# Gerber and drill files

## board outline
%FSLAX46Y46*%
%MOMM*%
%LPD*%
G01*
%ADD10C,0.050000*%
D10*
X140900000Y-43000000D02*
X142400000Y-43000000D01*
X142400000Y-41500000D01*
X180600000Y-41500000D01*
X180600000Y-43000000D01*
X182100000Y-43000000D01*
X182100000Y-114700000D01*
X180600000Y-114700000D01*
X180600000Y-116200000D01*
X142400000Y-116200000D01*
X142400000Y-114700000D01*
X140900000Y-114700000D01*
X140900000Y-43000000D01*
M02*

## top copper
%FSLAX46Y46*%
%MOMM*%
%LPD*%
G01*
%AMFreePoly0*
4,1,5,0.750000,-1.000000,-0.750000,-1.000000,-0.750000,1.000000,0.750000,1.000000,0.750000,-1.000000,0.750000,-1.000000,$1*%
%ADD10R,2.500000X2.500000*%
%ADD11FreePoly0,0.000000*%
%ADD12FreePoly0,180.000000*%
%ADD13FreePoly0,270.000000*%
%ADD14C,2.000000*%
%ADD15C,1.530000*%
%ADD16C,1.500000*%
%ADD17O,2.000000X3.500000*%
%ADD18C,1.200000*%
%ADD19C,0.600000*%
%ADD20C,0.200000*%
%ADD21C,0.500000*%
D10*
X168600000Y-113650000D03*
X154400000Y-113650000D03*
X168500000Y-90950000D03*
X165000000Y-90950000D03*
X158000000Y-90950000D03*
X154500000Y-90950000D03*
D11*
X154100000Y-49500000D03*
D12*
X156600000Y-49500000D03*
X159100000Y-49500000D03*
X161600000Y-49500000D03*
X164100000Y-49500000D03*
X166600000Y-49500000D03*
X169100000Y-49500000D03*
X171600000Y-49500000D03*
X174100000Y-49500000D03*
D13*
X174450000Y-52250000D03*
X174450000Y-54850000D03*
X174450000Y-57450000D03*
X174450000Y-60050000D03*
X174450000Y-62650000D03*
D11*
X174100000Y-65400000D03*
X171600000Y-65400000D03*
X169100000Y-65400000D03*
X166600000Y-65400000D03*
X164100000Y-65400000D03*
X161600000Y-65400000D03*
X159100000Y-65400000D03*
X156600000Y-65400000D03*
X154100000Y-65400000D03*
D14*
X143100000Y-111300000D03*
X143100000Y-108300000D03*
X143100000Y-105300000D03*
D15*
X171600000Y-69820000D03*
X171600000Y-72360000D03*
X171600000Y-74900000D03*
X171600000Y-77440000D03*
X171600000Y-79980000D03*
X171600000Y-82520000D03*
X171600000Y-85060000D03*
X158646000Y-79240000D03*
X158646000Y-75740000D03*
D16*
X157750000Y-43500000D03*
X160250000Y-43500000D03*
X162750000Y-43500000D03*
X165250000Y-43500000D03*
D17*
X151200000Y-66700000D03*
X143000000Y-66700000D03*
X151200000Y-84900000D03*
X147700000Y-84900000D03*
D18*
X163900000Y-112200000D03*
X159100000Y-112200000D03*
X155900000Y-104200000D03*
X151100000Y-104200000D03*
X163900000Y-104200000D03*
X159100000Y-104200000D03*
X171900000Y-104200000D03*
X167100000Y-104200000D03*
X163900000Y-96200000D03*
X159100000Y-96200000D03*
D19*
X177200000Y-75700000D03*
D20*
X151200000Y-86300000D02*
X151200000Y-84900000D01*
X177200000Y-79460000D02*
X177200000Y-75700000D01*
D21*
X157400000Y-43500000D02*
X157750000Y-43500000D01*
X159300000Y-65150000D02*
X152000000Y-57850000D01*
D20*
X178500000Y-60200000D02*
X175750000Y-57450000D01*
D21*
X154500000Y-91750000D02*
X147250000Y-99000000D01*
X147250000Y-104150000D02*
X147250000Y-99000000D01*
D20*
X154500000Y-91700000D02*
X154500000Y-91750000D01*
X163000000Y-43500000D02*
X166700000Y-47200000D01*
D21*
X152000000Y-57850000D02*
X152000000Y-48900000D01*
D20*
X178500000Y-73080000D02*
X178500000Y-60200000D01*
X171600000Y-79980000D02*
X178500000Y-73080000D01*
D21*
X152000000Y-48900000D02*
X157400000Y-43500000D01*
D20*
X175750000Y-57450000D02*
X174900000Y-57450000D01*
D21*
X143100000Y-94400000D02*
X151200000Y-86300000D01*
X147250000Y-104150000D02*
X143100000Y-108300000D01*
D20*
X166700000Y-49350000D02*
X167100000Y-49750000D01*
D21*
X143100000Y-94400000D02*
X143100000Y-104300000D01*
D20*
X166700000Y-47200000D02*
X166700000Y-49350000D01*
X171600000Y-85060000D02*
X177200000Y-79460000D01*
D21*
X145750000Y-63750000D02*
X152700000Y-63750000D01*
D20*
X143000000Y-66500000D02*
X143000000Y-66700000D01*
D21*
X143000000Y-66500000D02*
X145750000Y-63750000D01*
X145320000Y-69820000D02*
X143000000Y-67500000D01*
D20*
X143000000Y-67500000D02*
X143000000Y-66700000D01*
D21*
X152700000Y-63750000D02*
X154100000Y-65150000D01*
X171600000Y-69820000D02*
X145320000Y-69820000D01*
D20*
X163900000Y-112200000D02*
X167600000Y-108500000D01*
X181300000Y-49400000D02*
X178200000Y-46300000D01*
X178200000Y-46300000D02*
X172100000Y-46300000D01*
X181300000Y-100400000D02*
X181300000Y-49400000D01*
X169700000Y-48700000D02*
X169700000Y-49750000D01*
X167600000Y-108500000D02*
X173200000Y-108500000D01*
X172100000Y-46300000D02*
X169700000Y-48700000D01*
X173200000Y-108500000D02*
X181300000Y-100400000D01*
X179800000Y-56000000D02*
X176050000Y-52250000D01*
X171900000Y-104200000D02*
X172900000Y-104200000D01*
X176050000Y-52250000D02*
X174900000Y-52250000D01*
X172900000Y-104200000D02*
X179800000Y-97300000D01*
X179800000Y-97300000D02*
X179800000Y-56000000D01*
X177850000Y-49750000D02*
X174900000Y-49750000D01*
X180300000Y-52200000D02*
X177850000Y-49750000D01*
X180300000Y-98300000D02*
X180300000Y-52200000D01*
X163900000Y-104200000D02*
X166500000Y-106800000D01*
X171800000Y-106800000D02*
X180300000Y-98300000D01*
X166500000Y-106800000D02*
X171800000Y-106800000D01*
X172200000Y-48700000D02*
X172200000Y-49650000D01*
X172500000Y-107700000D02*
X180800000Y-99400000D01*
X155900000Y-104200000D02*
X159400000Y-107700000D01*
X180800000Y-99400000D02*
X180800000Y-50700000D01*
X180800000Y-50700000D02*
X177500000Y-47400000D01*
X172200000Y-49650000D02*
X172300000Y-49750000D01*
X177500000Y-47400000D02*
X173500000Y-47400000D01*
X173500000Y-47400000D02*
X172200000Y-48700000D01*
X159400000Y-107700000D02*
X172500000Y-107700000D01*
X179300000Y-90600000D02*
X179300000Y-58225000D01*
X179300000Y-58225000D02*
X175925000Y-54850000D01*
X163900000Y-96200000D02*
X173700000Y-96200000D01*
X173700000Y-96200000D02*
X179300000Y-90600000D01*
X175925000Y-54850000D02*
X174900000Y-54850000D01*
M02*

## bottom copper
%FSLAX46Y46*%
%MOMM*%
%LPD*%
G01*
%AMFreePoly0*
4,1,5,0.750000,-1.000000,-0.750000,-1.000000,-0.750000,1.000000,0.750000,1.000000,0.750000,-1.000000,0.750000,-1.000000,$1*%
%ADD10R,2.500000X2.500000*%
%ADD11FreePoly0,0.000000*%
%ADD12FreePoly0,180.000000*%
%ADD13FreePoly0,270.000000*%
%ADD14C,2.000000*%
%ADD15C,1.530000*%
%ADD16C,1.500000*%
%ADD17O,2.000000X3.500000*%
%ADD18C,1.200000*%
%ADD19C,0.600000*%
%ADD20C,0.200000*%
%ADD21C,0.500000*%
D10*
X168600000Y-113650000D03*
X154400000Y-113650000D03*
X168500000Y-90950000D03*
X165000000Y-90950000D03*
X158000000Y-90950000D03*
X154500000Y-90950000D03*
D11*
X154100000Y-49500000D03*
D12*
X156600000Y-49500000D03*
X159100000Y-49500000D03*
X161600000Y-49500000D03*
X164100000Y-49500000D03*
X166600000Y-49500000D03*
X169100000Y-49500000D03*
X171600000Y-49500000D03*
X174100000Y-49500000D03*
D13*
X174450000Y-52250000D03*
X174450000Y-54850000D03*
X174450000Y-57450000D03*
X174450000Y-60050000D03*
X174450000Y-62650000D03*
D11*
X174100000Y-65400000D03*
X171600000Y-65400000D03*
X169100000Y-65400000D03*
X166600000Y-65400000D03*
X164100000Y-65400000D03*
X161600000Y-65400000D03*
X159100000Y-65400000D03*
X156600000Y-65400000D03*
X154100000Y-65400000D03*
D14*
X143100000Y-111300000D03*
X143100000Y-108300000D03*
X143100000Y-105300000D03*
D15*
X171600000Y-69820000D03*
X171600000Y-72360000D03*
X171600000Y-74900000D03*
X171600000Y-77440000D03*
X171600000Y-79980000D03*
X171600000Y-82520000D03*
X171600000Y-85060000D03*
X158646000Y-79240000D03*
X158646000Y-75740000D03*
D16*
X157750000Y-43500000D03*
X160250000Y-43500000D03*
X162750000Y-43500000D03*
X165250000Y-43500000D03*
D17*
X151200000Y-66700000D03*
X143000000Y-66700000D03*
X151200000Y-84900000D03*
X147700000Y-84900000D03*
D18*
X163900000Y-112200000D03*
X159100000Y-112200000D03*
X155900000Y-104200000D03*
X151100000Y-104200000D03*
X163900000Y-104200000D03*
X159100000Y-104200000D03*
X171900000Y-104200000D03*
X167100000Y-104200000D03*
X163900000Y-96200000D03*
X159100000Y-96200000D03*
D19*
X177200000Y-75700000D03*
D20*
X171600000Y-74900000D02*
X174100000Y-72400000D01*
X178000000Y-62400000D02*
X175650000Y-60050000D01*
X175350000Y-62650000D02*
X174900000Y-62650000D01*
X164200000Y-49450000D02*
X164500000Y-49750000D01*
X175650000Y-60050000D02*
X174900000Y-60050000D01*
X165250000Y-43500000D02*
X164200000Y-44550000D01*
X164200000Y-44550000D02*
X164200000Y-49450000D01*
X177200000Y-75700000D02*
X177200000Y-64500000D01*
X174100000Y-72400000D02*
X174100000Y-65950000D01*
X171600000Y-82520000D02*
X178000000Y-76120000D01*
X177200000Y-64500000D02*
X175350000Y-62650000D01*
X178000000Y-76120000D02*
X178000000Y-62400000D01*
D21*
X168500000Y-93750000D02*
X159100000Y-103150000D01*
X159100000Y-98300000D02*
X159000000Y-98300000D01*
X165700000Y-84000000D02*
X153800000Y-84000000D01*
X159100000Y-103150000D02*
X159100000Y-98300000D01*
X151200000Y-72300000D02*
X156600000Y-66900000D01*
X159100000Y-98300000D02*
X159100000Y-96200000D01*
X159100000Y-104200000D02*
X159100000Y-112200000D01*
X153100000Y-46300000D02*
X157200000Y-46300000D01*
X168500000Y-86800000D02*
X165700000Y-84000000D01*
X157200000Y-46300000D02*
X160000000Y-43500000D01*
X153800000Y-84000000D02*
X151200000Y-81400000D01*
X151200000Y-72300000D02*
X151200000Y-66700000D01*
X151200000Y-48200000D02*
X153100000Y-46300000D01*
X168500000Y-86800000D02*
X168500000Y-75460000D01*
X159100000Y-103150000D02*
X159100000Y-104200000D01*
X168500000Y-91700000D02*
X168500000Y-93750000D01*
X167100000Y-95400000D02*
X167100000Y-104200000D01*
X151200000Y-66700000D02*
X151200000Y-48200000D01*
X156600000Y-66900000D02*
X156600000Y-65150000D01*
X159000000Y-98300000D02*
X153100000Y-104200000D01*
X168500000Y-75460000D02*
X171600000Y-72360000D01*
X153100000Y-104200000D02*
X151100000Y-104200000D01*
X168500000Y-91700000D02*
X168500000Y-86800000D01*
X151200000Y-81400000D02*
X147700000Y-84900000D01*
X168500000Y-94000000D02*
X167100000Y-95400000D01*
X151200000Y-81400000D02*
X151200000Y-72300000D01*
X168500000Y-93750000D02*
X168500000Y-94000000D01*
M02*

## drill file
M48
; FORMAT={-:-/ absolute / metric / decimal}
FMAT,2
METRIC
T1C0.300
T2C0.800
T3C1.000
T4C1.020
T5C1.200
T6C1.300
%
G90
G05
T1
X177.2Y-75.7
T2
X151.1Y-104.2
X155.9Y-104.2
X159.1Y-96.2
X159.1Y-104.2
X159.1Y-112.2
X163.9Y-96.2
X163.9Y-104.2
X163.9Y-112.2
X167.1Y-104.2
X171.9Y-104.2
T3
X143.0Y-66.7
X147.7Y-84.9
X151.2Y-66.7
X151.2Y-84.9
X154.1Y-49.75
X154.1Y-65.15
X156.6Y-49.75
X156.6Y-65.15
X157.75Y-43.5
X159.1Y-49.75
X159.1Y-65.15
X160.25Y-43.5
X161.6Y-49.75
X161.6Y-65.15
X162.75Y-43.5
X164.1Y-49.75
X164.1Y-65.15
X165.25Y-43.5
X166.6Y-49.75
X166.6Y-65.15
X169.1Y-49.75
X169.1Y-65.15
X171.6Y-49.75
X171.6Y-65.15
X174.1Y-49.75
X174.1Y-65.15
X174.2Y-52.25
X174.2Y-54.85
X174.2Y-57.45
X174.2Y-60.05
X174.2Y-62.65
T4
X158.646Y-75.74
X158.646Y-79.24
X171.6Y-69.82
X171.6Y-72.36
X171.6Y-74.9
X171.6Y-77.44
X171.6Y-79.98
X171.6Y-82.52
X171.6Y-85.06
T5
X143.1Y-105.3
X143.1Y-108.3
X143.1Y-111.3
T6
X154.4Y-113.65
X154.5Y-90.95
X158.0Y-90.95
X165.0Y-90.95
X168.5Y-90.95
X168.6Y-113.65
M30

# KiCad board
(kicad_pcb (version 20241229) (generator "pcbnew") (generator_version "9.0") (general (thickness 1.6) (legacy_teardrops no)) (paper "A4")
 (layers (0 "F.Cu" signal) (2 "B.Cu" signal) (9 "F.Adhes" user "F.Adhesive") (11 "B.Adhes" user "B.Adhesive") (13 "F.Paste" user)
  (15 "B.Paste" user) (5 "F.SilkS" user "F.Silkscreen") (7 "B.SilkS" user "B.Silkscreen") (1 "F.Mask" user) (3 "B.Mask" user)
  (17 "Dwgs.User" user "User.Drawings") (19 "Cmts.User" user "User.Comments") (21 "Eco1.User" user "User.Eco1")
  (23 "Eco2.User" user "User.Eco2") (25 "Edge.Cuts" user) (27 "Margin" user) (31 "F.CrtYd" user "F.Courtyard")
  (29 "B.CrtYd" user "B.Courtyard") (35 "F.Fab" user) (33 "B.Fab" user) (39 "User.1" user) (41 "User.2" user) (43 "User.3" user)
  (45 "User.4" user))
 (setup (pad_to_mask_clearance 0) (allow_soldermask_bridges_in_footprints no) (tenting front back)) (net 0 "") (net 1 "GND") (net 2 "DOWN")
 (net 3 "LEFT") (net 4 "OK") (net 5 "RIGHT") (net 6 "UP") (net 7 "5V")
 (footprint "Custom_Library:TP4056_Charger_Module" (layer "F.Cu") (at 161.5 101.9 180)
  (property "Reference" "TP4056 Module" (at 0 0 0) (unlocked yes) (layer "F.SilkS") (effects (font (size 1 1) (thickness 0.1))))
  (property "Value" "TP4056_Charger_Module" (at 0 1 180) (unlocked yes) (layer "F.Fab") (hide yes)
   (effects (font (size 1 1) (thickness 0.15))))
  (pad "1" thru_hole rect (at -7.1 -11.75 180) (size 2.5 2.5) (drill 1.3) (layers "*.Cu" "*.Mask") (remove_unused_layers no)
   (thermal_bridge_angle 45))
  (pad "2" thru_hole rect (at 7.1 -11.75 180) (size 2.5 2.5) (drill 1.3) (layers "*.Cu" "*.Mask") (remove_unused_layers no)
   (thermal_bridge_angle 45))
  (pad "3" thru_hole rect (at -7 10.95 180) (size 2.5 2.5) (drill 1.3) (layers "*.Cu" "*.Mask") (remove_unused_layers no) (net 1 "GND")
   (thermal_bridge_angle 45))
  (pad "4" thru_hole rect (at -3.5 10.95 180) (size 2.5 2.5) (drill 1.3) (layers "*.Cu" "*.Mask") (remove_unused_layers no)
   (thermal_bridge_angle 45))
  (pad "5" thru_hole rect (at 3.5 10.95 180) (size 2.5 2.5) (drill 1.3) (layers "*.Cu" "*.Mask") (remove_unused_layers no)
   (thermal_bridge_angle 45))
  (pad "6" thru_hole rect (at 7 10.95 180) (size 2.5 2.5) (drill 1.3) (layers "*.Cu" "*.Mask") (remove_unused_layers no)
   (thermal_bridge_angle 45))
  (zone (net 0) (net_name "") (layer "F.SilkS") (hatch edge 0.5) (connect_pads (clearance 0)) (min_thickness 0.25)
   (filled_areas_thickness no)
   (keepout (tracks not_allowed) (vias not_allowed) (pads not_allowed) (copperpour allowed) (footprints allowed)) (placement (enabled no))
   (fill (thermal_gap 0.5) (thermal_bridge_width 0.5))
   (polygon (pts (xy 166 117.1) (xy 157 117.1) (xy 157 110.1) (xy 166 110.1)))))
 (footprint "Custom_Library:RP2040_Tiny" (layer "F.Cu") (at 164.5 57.45)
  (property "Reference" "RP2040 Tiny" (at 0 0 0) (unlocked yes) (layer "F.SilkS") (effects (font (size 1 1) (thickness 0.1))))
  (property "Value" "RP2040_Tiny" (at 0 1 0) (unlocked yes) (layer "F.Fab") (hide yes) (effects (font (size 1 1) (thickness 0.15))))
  (pad "1" thru_hole custom (at -10.4 -7.7) (size 1.5 2) (drill 1 (offset 0 -0.25)) (layers "*.Cu" "*.Mask") (remove_unused_layers no)
   (options (clearance outline) (anchor rect)) (primitives))
  (pad "2" thru_hole custom (at -7.9 -7.7 180) (size 1.5 2) (drill 1 (offset 0 0.25)) (layers "*.Cu" "*.Mask") (remove_unused_layers no)
   (options (clearance outline) (anchor rect)) (primitives))
  (pad "3" thru_hole custom (at -5.4 -7.7 180) (size 1.5 2) (drill 1 (offset 0 0.25)) (layers "*.Cu" "*.Mask") (remove_unused_layers no)
   (options (clearance outline) (anchor rect)) (primitives))
  (pad "4" thru_hole custom (at -2.9 -7.7 180) (size 1.5 2) (drill 1 (offset 0 0.25)) (layers "*.Cu" "*.Mask") (remove_unused_layers no)
   (options (clearance outline) (anchor rect)) (primitives))
  (pad "5" thru_hole custom (at -0.4 -7.7 180) (size 1.5 2) (drill 1 (offset 0 0.25)) (layers "*.Cu" "*.Mask") (remove_unused_layers no)
   (options (clearance outline) (anchor rect)) (primitives))
  (pad "6" thru_hole custom (at 2.1 -7.7 180) (size 1.5 2) (drill 1 (offset 0 0.25)) (layers "*.Cu" "*.Mask") (remove_unused_layers no)
   (options (clearance outline) (anchor rect)) (primitives))
  (pad "7" thru_hole custom (at 4.6 -7.7 180) (size 1.5 2) (drill 1 (offset 0 0.25)) (layers "*.Cu" "*.Mask") (remove_unused_layers no)
   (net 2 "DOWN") (options (clearance outline) (anchor rect)) (primitives))
  (pad "8" thru_hole custom (at 7.1 -7.7 180) (size 1.5 2) (drill 1 (offset 0 0.25)) (layers "*.Cu" "*.Mask") (remove_unused_layers no)
   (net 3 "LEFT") (options (clearance outline) (anchor rect)) (primitives))
  (pad "9" thru_hole custom (at 9.6 -7.7 180) (size 1.5 2) (drill 1 (offset 0 0.25)) (layers "*.Cu" "*.Mask") (remove_unused_layers no)
   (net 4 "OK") (options (clearance outline) (anchor rect)) (primitives))
  (pad "10" thru_hole custom (at 9.7 -5.2 270) (size 1.5 2) (drill 1 (offset 0 -0.25)) (layers "*.Cu" "*.Mask") (remove_unused_layers no)
   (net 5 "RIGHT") (options (clearance outline) (anchor rect)) (primitives))
  (pad "11" thru_hole custom (at 9.7 -2.6 270) (size 1.5 2) (drill 1 (offset 0 -0.25)) (layers "*.Cu" "*.Mask") (remove_unused_layers no)
   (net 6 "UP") (options (clearance outline) (anchor rect)) (primitives))
  (pad "12" thru_hole custom (at 9.7 0 270) (size 1.5 2) (drill 1 (offset 0 -0.25)) (layers "*.Cu" "*.Mask") (remove_unused_layers no)
   (options (clearance outline) (anchor rect)) (primitives))
  (pad "13" thru_hole custom (at 9.7 2.6 270) (size 1.5 2) (drill 1 (offset 0 -0.25)) (layers "*.Cu" "*.Mask") (remove_unused_layers no)
   (options (clearance outline) (anchor rect)) (primitives))
  (pad "14" thru_hole custom (at 9.7 5.2 270) (size 1.5 2) (drill 1 (offset 0 -0.25)) (layers "*.Cu" "*.Mask") (remove_unused_layers no)
   (options (clearance outline) (anchor rect)) (primitives))
  (pad "15" thru_hole custom (at 9.6 7.7) (size 1.5 2) (drill 1 (offset 0 0.25)) (layers "*.Cu" "*.Mask") (remove_unused_layers no)
   (options (clearance outline) (anchor rect)) (primitives))
  (pad "16" thru_hole custom (at 7.1 7.7) (size 1.5 2) (drill 1 (offset 0 0.25)) (layers "*.Cu" "*.Mask") (remove_unused_layers no)
   (options (clearance outline) (anchor rect)) (primitives))
  (pad "17" thru_hole custom (at 4.6 7.7) (size 1.5 2) (drill 1 (offset 0 0.25)) (layers "*.Cu" "*.Mask") (remove_unused_layers no)
   (options (clearance outline) (anchor rect)) (primitives))
  (pad "18" thru_hole custom (at 2.1 7.7) (size 1.5 2) (drill 1 (offset 0 0.25)) (layers "*.Cu" "*.Mask") (remove_unused_layers no)
   (options (clearance outline) (anchor rect)) (primitives))
  (pad "19" thru_hole custom (at -0.4 7.7) (size 1.5 2) (drill 1 (offset 0 0.25)) (layers "*.Cu" "*.Mask") (remove_unused_layers no)
   (options (clearance outline) (anchor rect)) (primitives))
  (pad "20" thru_hole custom (at -2.9 7.7) (size 1.5 2) (drill 1 (offset 0 0.25)) (layers "*.Cu" "*.Mask") (remove_unused_layers no)
   (options (clearance outline) (anchor rect)) (primitives))
  (pad "21" thru_hole custom (at -5.4 7.7) (size 1.5 2) (drill 1 (offset 0 0.25)) (layers "*.Cu" "*.Mask") (remove_unused_layers no)
   (options (clearance outline) (anchor rect)) (primitives))
  (pad "22" thru_hole custom (at -7.9 7.7) (size 1.5 2) (drill 1 (offset 0 0.25)) (layers "*.Cu" "*.Mask") (remove_unused_layers no)
   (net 1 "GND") (options (clearance outline) (anchor rect)) (primitives))
  (pad "23" thru_hole custom (at -10.4 7.7) (size 1.5 2) (drill 1 (offset 0 0.25)) (layers "*.Cu" "*.Mask") (remove_unused_layers no)
   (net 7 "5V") (options (clearance outline) (anchor rect)) (primitives))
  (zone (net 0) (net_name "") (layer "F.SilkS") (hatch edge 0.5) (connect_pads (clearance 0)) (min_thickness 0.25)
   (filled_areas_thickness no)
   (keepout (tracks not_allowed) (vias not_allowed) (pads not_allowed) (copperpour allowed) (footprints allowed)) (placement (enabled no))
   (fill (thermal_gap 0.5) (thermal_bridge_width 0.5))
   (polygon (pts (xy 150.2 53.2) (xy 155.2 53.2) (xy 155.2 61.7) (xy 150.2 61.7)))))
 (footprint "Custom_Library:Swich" (layer "F.Cu") (at 143.1 108.3 90)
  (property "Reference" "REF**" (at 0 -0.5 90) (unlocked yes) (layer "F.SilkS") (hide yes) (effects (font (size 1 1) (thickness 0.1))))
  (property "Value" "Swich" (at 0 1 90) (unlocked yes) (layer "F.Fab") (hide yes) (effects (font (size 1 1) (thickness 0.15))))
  (pad "1" thru_hole circle (at -3 0 90) (size 2 2) (drill 1.2) (layers "*.Cu" "*.Mask") (remove_unused_layers no))
  (pad "2" thru_hole circle (at 0 0 90) (size 2 2) (drill 1.2) (layers "*.Cu" "*.Mask") (remove_unused_layers no))
  (pad "3" thru_hole circle (at 3 0 90) (size 2 2) (drill 1.2) (layers "*.Cu" "*.Mask") (remove_unused_layers no)))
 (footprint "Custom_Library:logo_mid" (layer "F.Cu") (at 177.5 100 90)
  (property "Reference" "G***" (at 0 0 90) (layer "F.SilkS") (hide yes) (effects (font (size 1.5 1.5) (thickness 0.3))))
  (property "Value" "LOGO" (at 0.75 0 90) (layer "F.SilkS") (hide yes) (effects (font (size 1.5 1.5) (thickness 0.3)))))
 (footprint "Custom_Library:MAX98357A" (layer "F.Cu") (at 164.615 77.25 90)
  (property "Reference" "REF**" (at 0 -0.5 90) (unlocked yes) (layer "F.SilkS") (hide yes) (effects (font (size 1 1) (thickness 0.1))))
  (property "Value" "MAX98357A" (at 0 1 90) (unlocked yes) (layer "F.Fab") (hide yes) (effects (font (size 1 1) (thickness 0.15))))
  (pad "JP1_1" thru_hole circle (at 7.43 6.985 90) (size 1.53 1.53) (drill 1.02) (layers "*.Cu" "*.Mask") (remove_unused_layers no)
   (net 7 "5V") (solder_mask_margin 0.102))
  (pad "JP1_2" thru_hole circle (at 4.89 6.985 90) (size 1.53 1.53) (drill 1.02) (layers "*.Cu" "*.Mask") (remove_unused_layers no)
   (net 1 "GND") (solder_mask_margin 0.102))
  (pad "JP1_3" thru_hole circle (at 2.35 6.985 90) (size 1.53 1.53) (drill 1.02) (layers "*.Cu" "*.Mask") (remove_unused_layers no)
   (solder_mask_margin 0.102))
  (pad "JP1_4" thru_hole circle (at -0.19 6.985 90) (size 1.53 1.53) (drill 1.02) (layers "*.Cu" "*.Mask") (remove_unused_layers no)
   (solder_mask_margin 0.102))
  (pad "JP1_5" thru_hole circle (at -2.73 6.985 90) (size 1.53 1.53) (drill 1.02) (layers "*.Cu" "*.Mask") (remove_unused_layers no)
   (solder_mask_margin 0.102))
  (pad "JP1_6" thru_hole circle (at -5.27 6.985 90) (size 1.53 1.53) (drill 1.02) (layers "*.Cu" "*.Mask") (remove_unused_layers no)
   (solder_mask_margin 0.102))
  (pad "JP1_7" thru_hole circle (at -7.81 6.985 90) (size 1.53 1.53) (drill 1.02) (layers "*.Cu" "*.Mask") (remove_unused_layers no)
   (solder_mask_margin 0.102))
  (pad "X1_1" thru_hole circle (at -1.99 -5.969 90) (size 1.53 1.53) (drill 1.02) (layers "*.Cu" "*.Mask") (remove_unused_layers no)
   (solder_mask_margin 0.102))
  (pad "X1_2" thru_hole circle (at 1.51 -5.969 90) (size 1.53 1.53) (drill 1.02) (layers "*.Cu" "*.Mask") (remove_unused_layers no)
   (solder_mask_margin 0.102)))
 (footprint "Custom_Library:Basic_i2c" (layer "F.Cu") (at 161.5 43.5)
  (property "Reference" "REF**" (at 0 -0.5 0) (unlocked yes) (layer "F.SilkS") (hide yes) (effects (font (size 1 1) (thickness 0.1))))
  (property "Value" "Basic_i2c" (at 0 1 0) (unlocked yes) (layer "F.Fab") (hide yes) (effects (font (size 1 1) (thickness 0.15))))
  (pad "1" thru_hole circle (at -3.75 0) (size 1.5 1.5) (drill 1) (layers "*.Cu" "*.Mask") (remove_unused_layers no))
  (pad "2" thru_hole circle (at -1.25 0) (size 1.5 1.5) (drill 1) (layers "*.Cu" "*.Mask") (remove_unused_layers no) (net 1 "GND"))
  (pad "3" thru_hole circle (at 1.25 0) (size 1.5 1.5) (drill 1) (layers "*.Cu" "*.Mask") (remove_unused_layers no))
  (pad "4" thru_hole circle (at 3.75 0) (size 1.5 1.5) (drill 1) (layers "*.Cu" "*.Mask") (remove_unused_layers no)))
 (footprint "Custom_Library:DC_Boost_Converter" (layer "F.Cu") (at 147.1 75.8 -90)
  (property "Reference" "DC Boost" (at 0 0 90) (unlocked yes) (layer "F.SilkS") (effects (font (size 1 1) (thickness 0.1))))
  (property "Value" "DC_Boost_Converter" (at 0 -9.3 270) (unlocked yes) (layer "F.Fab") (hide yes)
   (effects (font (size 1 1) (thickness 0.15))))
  (pad "1" thru_hole oval (at -9.1 -4.1) (size 2 3.5) (drill 1) (layers "*.Cu" "*.Mask") (remove_unused_layers no) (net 1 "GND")
   (thermal_bridge_angle 45))
  (pad "2" thru_hole oval (at -9.1 4.1) (size 2 3.5) (drill 1) (layers "*.Cu" "*.Mask") (remove_unused_layers no) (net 7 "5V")
   (thermal_bridge_angle 45))
  (pad "3" thru_hole oval (at 9.1 -4.1) (size 2 3.5) (drill 1) (layers "*.Cu" "*.Mask") (remove_unused_layers no) (thermal_bridge_angle 45))
  (pad "4" thru_hole oval (at 9.1 -0.6) (size 2 3.5) (drill 1) (layers "*.Cu" "*.Mask") (remove_unused_layers no) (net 1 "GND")
   (thermal_bridge_angle 45)))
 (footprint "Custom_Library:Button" (layer "B.Cu") (at 161.5 112.2 180)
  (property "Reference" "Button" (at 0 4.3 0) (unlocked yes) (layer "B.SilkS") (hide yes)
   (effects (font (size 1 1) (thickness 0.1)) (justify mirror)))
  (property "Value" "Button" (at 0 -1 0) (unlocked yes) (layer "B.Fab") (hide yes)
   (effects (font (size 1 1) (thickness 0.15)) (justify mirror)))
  (pad "1" thru_hole circle (at -2.4 0 180) (size 1.2 1.2) (drill 0.8) (layers "*.Cu" "*.Mask") (remove_unused_layers no) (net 2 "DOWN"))
  (pad "2" thru_hole circle (at 2.4 0 180) (size 1.2 1.2) (drill 0.8) (layers "*.Cu" "*.Mask") (remove_unused_layers no) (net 1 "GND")))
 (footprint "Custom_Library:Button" (layer "B.Cu") (at 153.5 104.2 180)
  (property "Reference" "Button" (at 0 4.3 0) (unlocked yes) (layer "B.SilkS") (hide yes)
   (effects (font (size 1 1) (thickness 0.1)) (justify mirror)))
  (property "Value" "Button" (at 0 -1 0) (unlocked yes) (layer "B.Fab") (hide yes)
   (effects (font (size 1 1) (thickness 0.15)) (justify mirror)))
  (pad "1" thru_hole circle (at -2.4 0 180) (size 1.2 1.2) (drill 0.8) (layers "*.Cu" "*.Mask") (remove_unused_layers no) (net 3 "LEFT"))
  (pad "2" thru_hole circle (at 2.4 0 180) (size 1.2 1.2) (drill 0.8) (layers "*.Cu" "*.Mask") (remove_unused_layers no) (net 1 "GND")))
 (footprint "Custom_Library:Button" (layer "B.Cu") (at 161.5 104.2 180)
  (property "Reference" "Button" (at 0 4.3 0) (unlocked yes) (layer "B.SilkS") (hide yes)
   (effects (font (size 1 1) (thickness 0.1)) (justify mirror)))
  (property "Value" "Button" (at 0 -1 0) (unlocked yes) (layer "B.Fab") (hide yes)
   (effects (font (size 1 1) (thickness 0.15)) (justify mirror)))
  (pad "1" thru_hole circle (at -2.4 0 180) (size 1.2 1.2) (drill 0.8) (layers "*.Cu" "*.Mask") (remove_unused_layers no) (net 4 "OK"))
  (pad "2" thru_hole circle (at 2.4 0 180) (size 1.2 1.2) (drill 0.8) (layers "*.Cu" "*.Mask") (remove_unused_layers no) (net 1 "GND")))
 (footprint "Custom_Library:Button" (layer "B.Cu") (at 169.5 104.2 180)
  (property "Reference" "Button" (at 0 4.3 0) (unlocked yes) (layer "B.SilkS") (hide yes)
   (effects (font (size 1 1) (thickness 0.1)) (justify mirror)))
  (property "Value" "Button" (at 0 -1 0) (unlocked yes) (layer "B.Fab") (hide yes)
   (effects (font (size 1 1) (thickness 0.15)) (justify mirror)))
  (pad "1" thru_hole circle (at -2.4 0 180) (size 1.2 1.2) (drill 0.8) (layers "*.Cu" "*.Mask") (remove_unused_layers no) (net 5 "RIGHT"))
  (pad "2" thru_hole circle (at 2.4 0 180) (size 1.2 1.2) (drill 0.8) (layers "*.Cu" "*.Mask") (remove_unused_layers no) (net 1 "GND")))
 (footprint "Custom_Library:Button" (layer "B.Cu") (at 161.5 96.2 180)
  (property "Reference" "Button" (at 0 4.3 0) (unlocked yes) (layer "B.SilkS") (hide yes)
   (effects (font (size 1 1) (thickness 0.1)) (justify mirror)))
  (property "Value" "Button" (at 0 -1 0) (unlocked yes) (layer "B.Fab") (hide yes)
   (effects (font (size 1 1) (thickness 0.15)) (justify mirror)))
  (pad "1" thru_hole circle (at -2.4 0 180) (size 1.2 1.2) (drill 0.8) (layers "*.Cu" "*.Mask") (remove_unused_layers no) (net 6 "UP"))
  (pad "2" thru_hole circle (at 2.4 0 180) (size 1.2 1.2) (drill 0.8) (layers "*.Cu" "*.Mask") (remove_unused_layers no) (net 1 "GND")))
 (gr_poly
  (pts (xy 140.9 43) (xy 142.4 43) (xy 142.4 41.5) (xy 180.6 41.5) (xy 180.6 43) (xy 182.1 43) (xy 182.1 114.7) (xy 180.6 114.7)
   (xy 180.6 116.2) (xy 142.4 116.2) (xy 142.4 114.7) (xy 140.9 114.7))
  (stroke (width 0.05) (type solid)) (fill no) (layer "Edge.Cuts"))
 (segment (start 151.2 86.3) (end 151.2 84.9) (width 0.2) (layer "F.Cu") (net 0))
 (segment (start 177.2 79.46) (end 177.2 75.7) (width 0.2) (layer "F.Cu") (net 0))
 (segment (start 157.4 43.5) (end 157.75 43.5) (width 0.5) (layer "F.Cu") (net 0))
 (segment (start 159.3 65.15) (end 152 57.85) (width 0.5) (layer "F.Cu") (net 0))
 (segment (start 178.5 60.2) (end 175.75 57.45) (width 0.2) (layer "F.Cu") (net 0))
 (segment (start 154.5 91.75) (end 147.25 99) (width 0.5) (layer "F.Cu") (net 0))
 (segment (start 147.25 104.15) (end 147.25 99) (width 0.5) (layer "F.Cu") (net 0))
 (segment (start 154.5 91.7) (end 154.5 91.75) (width 0.2) (layer "F.Cu") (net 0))
 (segment (start 163 43.5) (end 166.7 47.2) (width 0.2) (layer "F.Cu") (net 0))
 (segment (start 152 57.85) (end 152 48.9) (width 0.5) (layer "F.Cu") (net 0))
 (segment (start 178.5 73.08) (end 178.5 60.2) (width 0.2) (layer "F.Cu") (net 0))
 (segment (start 171.6 79.98) (end 178.5 73.08) (width 0.2) (layer "F.Cu") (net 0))
 (segment (start 152 48.9) (end 157.4 43.5) (width 0.5) (layer "F.Cu") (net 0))
 (segment (start 175.75 57.45) (end 174.9 57.45) (width 0.2) (layer "F.Cu") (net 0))
 (segment (start 143.1 94.4) (end 151.2 86.3) (width 0.5) (layer "F.Cu") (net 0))
 (segment (start 147.25 104.15) (end 143.1 108.3) (width 0.5) (layer "F.Cu") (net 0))
 (segment (start 166.7 49.35) (end 167.1 49.75) (width 0.2) (layer "F.Cu") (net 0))
 (segment (start 143.1 94.4) (end 143.1 104.3) (width 0.5) (layer "F.Cu") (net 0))
 (segment (start 166.7 47.2) (end 166.7 49.35) (width 0.2) (layer "F.Cu") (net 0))
 (segment (start 171.6 85.06) (end 177.2 79.46) (width 0.2) (layer "F.Cu") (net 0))
 (via (at 177.2 75.7) (size 0.6) (drill 0.3) (layers "F.Cu" "B.Cu") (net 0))
 (segment (start 171.6 74.9) (end 174.1 72.4) (width 0.2) (layer "B.Cu") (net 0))
 (segment (start 178 62.4) (end 175.65 60.05) (width 0.2) (layer "B.Cu") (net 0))
 (segment (start 175.35 62.65) (end 174.9 62.65) (width 0.2) (layer "B.Cu") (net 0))
 (segment (start 164.2 49.45) (end 164.5 49.75) (width 0.2) (layer "B.Cu") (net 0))
 (segment (start 175.65 60.05) (end 174.9 60.05) (width 0.2) (layer "B.Cu") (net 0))
 (segment (start 165.25 43.5) (end 164.2 44.55) (width 0.2) (layer "B.Cu") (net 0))
 (segment (start 164.2 44.55) (end 164.2 49.45) (width 0.2) (layer "B.Cu") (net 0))
 (segment (start 177.2 75.7) (end 177.2 64.5) (width 0.2) (layer "B.Cu") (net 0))
 (segment (start 174.1 72.4) (end 174.1 65.95) (width 0.2) (layer "B.Cu") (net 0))
 (segment (start 171.6 82.52) (end 178 76.12) (width 0.2) (layer "B.Cu") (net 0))
 (segment (start 177.2 64.5) (end 175.35 62.65) (width 0.2) (layer "B.Cu") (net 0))
 (segment (start 178 76.12) (end 178 62.4) (width 0.2) (layer "B.Cu") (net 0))
 (segment (start 168.5 93.75) (end 159.1 103.15) (width 0.5) (layer "B.Cu") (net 1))
 (segment (start 159.1 98.3) (end 159 98.3) (width 0.5) (layer "B.Cu") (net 1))
 (segment (start 165.7 84) (end 153.8 84) (width 0.5) (layer "B.Cu") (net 1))
 (segment (start 159.1 103.15) (end 159.1 98.3) (width 0.5) (layer "B.Cu") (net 1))
 (segment (start 151.2 72.3) (end 156.6 66.9) (width 0.5) (layer "B.Cu") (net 1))
 (segment (start 159.1 98.3) (end 159.1 96.2) (width 0.5) (layer "B.Cu") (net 1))
 (segment (start 159.1 104.2) (end 159.1 112.2) (width 0.5) (layer "B.Cu") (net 1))
 (segment (start 153.1 46.3) (end 157.2 46.3) (width 0.5) (layer "B.Cu") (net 1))
 (segment (start 168.5 86.8) (end 165.7 84) (width 0.5) (layer "B.Cu") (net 1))
 (segment (start 157.2 46.3) (end 160 43.5) (width 0.5) (layer "B.Cu") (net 1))
 (segment (start 153.8 84) (end 151.2 81.4) (width 0.5) (layer "B.Cu") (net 1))
 (segment (start 151.2 72.3) (end 151.2 66.7) (width 0.5) (layer "B.Cu") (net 1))
 (segment (start 151.2 48.2) (end 153.1 46.3) (width 0.5) (layer "B.Cu") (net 1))
 (segment (start 168.5 86.8) (end 168.5 75.46) (width 0.5) (layer "B.Cu") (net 1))
 (segment (start 159.1 103.15) (end 159.1 104.2) (width 0.5) (layer "B.Cu") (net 1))
 (segment (start 168.5 91.7) (end 168.5 93.75) (width 0.5) (layer "B.Cu") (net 1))
 (segment (start 167.1 95.4) (end 167.1 104.2) (width 0.5) (layer "B.Cu") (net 1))
 (segment (start 151.2 66.7) (end 151.2 48.2) (width 0.5) (layer "B.Cu") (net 1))
 (segment (start 156.6 66.9) (end 156.6 65.15) (width 0.5) (layer "B.Cu") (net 1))
 (segment (start 159 98.3) (end 153.1 104.2) (width 0.5) (layer "B.Cu") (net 1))
 (segment (start 168.5 75.46) (end 171.6 72.36) (width 0.5) (layer "B.Cu") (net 1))
 (segment (start 153.1 104.2) (end 151.1 104.2) (width 0.5) (layer "B.Cu") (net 1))
 (segment (start 168.5 91.7) (end 168.5 86.8) (width 0.5) (layer "B.Cu") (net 1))
 (segment (start 151.2 81.4) (end 147.7 84.9) (width 0.5) (layer "B.Cu") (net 1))
 (segment (start 168.5 94) (end 167.1 95.4) (width 0.5) (layer "B.Cu") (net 1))
 (segment (start 151.2 81.4) (end 151.2 72.3) (width 0.5) (layer "B.Cu") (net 1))
 (segment (start 168.5 93.75) (end 168.5 94) (width 0.5) (layer "B.Cu") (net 1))
 (segment (start 145.75 63.75) (end 152.7 63.75) (width 0.5) (layer "F.Cu") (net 7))
 (segment (start 143 66.5) (end 143 66.7) (width 0.2) (layer "F.Cu") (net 7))
 (segment (start 143 66.5) (end 145.75 63.75) (width 0.5) (layer "F.Cu") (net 7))
 (segment (start 145.32 69.82) (end 143 67.5) (width 0.5) (layer "F.Cu") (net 7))
 (segment (start 143 67.5) (end 143 66.7) (width 0.2) (layer "F.Cu") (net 7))
 (segment (start 152.7 63.75) (end 154.1 65.15) (width 0.5) (layer "F.Cu") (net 7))
 (segment (start 171.6 69.82) (end 145.32 69.82) (width 0.5) (layer "F.Cu") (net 7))
 (segment (start 163.9 112.2) (end 167.6 108.5) (width 0.2) (layer "F.Cu") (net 2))
 (segment (start 181.3 49.4) (end 178.2 46.3) (width 0.2) (layer "F.Cu") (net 2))
 (segment (start 178.2 46.3) (end 172.1 46.3) (width 0.2) (layer "F.Cu") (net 2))
 (segment (start 181.3 100.4) (end 181.3 49.4) (width 0.2) (layer "F.Cu") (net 2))
 (segment (start 169.7 48.7) (end 169.7 49.75) (width 0.2) (layer "F.Cu") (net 2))
 (segment (start 167.6 108.5) (end 173.2 108.5) (width 0.2) (layer "F.Cu") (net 2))
 (segment (start 172.1 46.3) (end 169.7 48.7) (width 0.2) (layer "F.Cu") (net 2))
 (segment (start 173.2 108.5) (end 181.3 100.4) (width 0.2) (layer "F.Cu") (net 2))
 (segment (start 179.8 56) (end 176.05 52.25) (width 0.2) (layer "F.Cu") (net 5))
 (segment (start 171.9 104.2) (end 172.9 104.2) (width 0.2) (layer "F.Cu") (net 5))
 (segment (start 176.05 52.25) (end 174.9 52.25) (width 0.2) (layer "F.Cu") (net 5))
 (segment (start 172.9 104.2) (end 179.8 97.3) (width 0.2) (layer "F.Cu") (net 5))
 (segment (start 179.8 97.3) (end 179.8 56) (width 0.2) (layer "F.Cu") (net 5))
 (segment (start 177.85 49.75) (end 174.9 49.75) (width 0.2) (layer "F.Cu") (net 4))
 (segment (start 180.3 52.2) (end 177.85 49.75) (width 0.2) (layer "F.Cu") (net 4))
 (segment (start 180.3 98.3) (end 180.3 52.2) (width 0.2) (layer "F.Cu") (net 4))
 (segment (start 163.9 104.2) (end 166.5 106.8) (width 0.2) (layer "F.Cu") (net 4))
 (segment (start 171.8 106.8) (end 180.3 98.3) (width 0.2) (layer "F.Cu") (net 4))
 (segment (start 166.5 106.8) (end 171.8 106.8) (width 0.2) (layer "F.Cu") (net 4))
 (segment (start 172.2 48.7) (end 172.2 49.65) (width 0.2) (layer "F.Cu") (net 3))
 (segment (start 172.5 107.7) (end 180.8 99.4) (width 0.2) (layer "F.Cu") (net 3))
 (segment (start 155.9 104.2) (end 159.4 107.7) (width 0.2) (layer "F.Cu") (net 3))
 (segment (start 180.8 99.4) (end 180.8 50.7) (width 0.2) (layer "F.Cu") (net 3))
 (segment (start 180.8 50.7) (end 177.5 47.4) (width 0.2) (layer "F.Cu") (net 3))
 (segment (start 172.2 49.65) (end 172.3 49.75) (width 0.2) (layer "F.Cu") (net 3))
 (segment (start 177.5 47.4) (end 173.5 47.4) (width 0.2) (layer "F.Cu") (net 3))
 (segment (start 173.5 47.4) (end 172.2 48.7) (width 0.2) (layer "F.Cu") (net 3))
 (segment (start 159.4 107.7) (end 172.5 107.7) (width 0.2) (layer "F.Cu") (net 3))
 (segment (start 179.3 90.6) (end 179.3 58.225) (width 0.2) (layer "F.Cu") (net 6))
 (segment (start 179.3 58.225) (end 175.925 54.85) (width 0.2) (layer "F.Cu") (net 6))
 (segment (start 163.9 96.2) (end 173.7 96.2) (width 0.2) (layer "F.Cu") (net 6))
 (segment (start 173.7 96.2) (end 179.3 90.6) (width 0.2) (layer "F.Cu") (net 6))
 (segment (start 175.925 54.85) (end 174.9 54.85) (width 0.2) (layer "F.Cu") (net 6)))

